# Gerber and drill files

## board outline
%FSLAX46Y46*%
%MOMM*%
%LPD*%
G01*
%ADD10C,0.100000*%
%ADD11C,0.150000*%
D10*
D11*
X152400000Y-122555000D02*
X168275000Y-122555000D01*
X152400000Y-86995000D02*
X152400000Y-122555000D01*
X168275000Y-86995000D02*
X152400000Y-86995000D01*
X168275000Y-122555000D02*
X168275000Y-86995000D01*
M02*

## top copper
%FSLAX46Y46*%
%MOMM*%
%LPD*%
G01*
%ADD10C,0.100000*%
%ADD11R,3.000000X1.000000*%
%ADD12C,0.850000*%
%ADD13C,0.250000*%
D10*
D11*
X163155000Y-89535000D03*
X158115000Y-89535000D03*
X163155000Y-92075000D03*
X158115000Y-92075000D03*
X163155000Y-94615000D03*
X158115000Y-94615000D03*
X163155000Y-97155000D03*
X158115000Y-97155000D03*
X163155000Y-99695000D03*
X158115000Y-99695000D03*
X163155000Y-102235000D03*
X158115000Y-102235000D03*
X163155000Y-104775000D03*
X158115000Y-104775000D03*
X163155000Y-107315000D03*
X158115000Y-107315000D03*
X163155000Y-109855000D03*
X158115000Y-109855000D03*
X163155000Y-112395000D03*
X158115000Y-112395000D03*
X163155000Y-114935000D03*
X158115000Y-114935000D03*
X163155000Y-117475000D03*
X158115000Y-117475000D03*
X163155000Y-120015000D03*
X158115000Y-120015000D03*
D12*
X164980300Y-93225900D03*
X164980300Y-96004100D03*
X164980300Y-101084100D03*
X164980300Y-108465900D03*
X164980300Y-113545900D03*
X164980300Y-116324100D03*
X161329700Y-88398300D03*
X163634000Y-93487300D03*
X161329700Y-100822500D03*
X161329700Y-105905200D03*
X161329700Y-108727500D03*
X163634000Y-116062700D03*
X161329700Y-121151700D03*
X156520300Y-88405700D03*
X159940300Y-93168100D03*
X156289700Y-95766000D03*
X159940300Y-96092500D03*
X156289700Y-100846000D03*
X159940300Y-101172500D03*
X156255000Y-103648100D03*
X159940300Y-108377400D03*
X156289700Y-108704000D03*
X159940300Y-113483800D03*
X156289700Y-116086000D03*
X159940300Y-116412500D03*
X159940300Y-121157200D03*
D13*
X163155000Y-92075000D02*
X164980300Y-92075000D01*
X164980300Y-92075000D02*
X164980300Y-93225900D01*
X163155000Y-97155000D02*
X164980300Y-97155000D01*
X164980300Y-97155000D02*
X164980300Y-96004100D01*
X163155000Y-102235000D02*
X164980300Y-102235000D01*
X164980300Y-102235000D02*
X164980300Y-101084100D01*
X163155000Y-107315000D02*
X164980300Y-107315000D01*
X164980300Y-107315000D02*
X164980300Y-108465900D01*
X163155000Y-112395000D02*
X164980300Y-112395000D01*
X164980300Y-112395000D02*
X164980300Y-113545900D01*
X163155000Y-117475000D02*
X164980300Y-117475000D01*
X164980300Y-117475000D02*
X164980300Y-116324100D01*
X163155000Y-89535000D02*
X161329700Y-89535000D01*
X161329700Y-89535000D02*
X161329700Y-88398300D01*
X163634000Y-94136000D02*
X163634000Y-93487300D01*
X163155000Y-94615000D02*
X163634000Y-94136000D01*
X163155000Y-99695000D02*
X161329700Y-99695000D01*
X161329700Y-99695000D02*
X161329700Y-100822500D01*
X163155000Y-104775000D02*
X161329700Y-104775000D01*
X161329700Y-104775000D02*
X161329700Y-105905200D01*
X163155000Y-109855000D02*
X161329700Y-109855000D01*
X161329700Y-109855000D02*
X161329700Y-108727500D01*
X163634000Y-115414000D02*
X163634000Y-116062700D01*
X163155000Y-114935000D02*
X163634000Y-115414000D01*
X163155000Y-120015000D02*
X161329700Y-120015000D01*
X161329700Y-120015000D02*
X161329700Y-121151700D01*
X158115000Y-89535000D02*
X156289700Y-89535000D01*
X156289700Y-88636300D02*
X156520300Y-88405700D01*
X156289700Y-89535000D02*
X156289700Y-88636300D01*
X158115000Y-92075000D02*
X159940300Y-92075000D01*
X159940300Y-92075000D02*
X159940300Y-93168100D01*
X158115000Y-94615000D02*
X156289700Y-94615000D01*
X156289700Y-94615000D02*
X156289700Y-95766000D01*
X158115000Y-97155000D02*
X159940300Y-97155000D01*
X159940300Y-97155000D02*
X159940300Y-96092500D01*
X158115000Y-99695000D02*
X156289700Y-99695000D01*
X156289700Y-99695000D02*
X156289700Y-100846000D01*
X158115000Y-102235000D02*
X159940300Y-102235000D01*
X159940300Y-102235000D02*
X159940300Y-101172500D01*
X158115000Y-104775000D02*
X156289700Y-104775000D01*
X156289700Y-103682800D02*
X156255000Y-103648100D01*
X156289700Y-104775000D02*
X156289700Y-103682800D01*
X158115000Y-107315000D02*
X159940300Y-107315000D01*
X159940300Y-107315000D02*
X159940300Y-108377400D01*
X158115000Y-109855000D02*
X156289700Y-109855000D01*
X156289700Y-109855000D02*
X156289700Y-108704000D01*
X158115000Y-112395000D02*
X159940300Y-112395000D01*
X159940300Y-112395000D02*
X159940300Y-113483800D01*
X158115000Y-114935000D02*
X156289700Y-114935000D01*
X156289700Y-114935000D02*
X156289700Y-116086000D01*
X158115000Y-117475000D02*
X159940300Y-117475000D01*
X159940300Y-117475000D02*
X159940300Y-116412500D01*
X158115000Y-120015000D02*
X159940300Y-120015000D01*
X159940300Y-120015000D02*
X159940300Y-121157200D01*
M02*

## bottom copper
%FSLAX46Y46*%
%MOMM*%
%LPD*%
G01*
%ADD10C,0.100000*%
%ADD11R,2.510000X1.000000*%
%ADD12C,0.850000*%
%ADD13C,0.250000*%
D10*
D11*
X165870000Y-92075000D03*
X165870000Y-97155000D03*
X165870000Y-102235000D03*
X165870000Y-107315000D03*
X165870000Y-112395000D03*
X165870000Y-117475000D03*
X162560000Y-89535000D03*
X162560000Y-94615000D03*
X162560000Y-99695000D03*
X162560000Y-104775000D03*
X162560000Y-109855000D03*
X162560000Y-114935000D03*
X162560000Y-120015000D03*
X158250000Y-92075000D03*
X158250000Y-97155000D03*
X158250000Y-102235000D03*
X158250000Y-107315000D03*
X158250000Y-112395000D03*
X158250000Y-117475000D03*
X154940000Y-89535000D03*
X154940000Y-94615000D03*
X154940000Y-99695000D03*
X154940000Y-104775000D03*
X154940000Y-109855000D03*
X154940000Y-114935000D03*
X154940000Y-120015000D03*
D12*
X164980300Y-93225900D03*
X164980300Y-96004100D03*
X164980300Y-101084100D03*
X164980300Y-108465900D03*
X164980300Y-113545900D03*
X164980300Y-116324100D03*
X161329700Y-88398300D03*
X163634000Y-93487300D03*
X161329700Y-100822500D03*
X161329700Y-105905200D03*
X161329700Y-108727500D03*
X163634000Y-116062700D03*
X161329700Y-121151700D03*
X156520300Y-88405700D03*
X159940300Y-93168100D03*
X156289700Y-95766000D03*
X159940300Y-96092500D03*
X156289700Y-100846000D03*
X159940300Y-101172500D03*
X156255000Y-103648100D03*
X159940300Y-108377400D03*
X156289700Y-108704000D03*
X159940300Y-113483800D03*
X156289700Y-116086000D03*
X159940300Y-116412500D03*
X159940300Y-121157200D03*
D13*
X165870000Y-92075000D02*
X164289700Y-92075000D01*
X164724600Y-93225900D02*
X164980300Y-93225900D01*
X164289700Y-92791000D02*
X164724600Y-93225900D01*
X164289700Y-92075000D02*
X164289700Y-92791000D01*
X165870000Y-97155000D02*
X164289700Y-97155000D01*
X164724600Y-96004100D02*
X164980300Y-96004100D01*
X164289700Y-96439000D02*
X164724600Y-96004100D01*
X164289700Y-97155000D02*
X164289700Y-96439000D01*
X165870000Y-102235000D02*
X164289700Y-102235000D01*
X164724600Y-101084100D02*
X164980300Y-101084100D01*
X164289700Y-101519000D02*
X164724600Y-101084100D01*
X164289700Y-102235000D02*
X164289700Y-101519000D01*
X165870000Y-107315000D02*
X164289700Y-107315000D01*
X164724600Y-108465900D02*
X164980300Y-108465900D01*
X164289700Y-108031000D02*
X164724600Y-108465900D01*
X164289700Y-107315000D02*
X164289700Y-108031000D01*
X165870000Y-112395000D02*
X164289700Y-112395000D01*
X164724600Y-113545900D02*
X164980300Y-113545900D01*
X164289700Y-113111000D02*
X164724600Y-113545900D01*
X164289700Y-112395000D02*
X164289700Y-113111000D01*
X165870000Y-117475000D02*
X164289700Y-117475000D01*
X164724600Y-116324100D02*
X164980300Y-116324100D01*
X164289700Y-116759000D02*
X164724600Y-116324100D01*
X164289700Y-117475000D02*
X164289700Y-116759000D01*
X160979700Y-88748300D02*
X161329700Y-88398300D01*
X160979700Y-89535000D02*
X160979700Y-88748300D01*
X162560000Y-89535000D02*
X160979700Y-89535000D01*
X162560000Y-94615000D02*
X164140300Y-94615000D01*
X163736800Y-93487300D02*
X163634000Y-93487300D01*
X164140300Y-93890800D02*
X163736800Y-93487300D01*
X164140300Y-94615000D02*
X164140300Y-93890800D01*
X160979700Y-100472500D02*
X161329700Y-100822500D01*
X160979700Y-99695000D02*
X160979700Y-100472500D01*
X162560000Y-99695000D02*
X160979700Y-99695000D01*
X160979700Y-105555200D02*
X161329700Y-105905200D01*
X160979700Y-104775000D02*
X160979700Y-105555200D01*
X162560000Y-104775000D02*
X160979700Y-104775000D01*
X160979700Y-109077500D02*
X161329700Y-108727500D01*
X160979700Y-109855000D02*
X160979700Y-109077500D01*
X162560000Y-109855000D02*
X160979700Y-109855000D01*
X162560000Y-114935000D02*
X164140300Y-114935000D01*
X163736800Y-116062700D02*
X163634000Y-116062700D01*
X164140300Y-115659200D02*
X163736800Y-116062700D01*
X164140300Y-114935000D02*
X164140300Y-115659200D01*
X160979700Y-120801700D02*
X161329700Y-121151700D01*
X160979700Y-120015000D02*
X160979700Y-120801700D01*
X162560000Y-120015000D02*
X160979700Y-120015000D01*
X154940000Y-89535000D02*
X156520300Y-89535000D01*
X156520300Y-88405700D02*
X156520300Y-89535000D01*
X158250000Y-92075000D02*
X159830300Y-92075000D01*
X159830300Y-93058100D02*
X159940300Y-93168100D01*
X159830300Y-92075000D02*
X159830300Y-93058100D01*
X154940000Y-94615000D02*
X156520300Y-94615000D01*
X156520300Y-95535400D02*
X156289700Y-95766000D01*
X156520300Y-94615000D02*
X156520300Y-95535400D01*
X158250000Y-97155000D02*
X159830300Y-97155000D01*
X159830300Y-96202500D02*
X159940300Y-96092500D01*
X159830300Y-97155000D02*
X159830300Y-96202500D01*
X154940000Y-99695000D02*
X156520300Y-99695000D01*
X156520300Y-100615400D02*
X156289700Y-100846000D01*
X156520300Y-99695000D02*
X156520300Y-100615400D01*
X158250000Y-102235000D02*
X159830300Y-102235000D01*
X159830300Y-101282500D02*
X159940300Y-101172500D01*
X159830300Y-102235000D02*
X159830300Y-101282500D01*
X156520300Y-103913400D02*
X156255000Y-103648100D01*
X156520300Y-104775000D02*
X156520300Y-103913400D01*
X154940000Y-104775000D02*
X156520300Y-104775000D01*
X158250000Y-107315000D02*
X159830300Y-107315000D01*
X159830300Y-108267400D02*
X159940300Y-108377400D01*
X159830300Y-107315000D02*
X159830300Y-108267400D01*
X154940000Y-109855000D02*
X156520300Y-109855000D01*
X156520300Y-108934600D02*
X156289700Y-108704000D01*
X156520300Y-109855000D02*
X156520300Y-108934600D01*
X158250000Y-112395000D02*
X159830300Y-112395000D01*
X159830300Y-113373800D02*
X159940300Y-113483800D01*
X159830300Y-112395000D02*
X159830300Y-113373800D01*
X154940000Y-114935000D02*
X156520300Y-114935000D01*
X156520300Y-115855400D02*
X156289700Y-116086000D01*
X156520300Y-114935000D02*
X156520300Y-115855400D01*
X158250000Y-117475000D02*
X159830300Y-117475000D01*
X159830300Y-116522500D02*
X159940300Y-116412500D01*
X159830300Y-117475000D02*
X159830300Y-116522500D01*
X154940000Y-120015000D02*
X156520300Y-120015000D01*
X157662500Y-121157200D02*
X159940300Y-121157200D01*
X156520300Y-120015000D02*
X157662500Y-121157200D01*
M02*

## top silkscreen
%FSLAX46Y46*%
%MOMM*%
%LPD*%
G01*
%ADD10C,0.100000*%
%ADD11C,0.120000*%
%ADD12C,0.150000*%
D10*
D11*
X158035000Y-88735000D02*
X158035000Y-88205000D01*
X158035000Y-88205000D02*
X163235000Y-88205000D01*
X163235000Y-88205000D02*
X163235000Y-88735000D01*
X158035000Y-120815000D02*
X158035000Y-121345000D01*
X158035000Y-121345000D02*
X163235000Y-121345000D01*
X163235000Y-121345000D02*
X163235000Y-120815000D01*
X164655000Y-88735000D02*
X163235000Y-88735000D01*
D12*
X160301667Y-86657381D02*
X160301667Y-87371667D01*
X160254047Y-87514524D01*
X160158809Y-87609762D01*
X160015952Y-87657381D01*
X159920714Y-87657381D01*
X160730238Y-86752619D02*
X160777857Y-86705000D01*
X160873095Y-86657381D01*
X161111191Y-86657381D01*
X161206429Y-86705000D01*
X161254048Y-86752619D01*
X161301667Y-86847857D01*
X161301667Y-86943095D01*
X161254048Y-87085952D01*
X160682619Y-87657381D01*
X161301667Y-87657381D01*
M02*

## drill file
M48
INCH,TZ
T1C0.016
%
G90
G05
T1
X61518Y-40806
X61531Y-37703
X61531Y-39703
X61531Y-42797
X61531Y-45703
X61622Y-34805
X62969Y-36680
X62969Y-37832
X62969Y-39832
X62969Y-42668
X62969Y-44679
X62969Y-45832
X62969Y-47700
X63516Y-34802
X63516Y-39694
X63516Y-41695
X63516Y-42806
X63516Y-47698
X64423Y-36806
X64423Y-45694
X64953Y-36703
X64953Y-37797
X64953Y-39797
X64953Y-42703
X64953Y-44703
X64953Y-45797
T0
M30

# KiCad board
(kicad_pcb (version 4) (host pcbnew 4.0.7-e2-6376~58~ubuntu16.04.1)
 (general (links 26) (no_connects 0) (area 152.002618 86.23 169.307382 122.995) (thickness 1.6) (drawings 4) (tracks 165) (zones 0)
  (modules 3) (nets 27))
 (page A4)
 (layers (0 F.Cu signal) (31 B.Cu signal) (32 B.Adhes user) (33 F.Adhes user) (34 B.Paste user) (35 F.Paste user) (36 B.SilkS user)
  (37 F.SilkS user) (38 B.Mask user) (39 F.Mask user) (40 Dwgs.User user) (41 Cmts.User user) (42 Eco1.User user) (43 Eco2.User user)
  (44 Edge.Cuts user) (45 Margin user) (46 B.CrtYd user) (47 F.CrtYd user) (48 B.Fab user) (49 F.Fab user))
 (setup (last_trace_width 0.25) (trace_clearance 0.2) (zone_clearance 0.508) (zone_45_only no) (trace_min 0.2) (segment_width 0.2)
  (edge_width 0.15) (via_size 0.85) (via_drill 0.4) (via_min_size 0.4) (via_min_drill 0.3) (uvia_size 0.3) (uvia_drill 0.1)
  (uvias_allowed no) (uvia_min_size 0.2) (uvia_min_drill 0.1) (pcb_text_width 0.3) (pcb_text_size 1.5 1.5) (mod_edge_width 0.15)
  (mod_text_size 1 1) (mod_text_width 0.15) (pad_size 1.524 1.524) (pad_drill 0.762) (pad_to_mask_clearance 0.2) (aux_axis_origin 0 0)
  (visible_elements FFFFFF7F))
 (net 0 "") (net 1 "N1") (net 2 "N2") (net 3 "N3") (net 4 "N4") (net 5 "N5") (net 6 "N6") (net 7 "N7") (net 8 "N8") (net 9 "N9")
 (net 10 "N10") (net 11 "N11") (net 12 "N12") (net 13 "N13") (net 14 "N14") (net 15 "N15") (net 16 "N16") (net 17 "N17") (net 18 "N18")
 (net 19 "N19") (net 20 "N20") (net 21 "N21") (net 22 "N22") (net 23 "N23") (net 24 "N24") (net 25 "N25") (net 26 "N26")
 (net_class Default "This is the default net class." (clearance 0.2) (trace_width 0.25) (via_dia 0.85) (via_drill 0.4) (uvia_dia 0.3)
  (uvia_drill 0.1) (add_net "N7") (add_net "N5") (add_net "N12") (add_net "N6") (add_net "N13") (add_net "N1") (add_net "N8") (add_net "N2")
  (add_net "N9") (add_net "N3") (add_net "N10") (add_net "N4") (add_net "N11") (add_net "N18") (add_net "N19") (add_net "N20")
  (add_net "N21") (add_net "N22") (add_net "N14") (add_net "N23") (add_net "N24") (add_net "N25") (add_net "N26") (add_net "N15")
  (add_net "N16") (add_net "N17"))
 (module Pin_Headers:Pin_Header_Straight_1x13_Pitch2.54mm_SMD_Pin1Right (layer B.Cu) (at 164.215 104.775 180)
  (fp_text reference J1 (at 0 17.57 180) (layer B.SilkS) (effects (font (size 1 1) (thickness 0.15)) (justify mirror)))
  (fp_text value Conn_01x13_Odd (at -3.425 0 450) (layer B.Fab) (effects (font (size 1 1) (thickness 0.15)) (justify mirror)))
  (pad 2 smd rect (at -1.655 12.7 180) (size 2.51 1) (layers B.Cu B.Paste B.Mask) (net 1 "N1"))
  (pad 4 smd rect (at -1.655 7.62 180) (size 2.51 1) (layers B.Cu B.Paste B.Mask) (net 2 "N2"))
  (pad 6 smd rect (at -1.655 2.54 180) (size 2.51 1) (layers B.Cu B.Paste B.Mask) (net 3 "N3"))
  (pad 8 smd rect (at -1.655 -2.54 180) (size 2.51 1) (layers B.Cu B.Paste B.Mask) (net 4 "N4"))
  (pad 10 smd rect (at -1.655 -7.62 180) (size 2.51 1) (layers B.Cu B.Paste B.Mask) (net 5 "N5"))
  (pad 12 smd rect (at -1.655 -12.7 180) (size 2.51 1) (layers B.Cu B.Paste B.Mask) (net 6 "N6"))
  (pad 1 smd rect (at 1.655 15.24 180) (size 2.51 1) (layers B.Cu B.Paste B.Mask) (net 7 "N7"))
  (pad 3 smd rect (at 1.655 10.16 180) (size 2.51 1) (layers B.Cu B.Paste B.Mask) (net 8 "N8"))
  (pad 5 smd rect (at 1.655 5.08 180) (size 2.51 1) (layers B.Cu B.Paste B.Mask) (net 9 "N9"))
  (pad 7 smd rect (at 1.655 0 180) (size 2.51 1) (layers B.Cu B.Paste B.Mask) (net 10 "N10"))
  (pad 9 smd rect (at 1.655 -5.08 180) (size 2.51 1) (layers B.Cu B.Paste B.Mask) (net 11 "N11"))
  (pad 11 smd rect (at 1.655 -10.16 180) (size 2.51 1) (layers B.Cu B.Paste B.Mask) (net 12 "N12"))
  (pad 13 smd rect (at 1.655 -15.24 180) (size 2.51 1) (layers B.Cu B.Paste B.Mask) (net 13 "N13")))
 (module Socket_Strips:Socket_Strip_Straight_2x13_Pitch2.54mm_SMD (layer F.Cu) (at 160.635 104.775)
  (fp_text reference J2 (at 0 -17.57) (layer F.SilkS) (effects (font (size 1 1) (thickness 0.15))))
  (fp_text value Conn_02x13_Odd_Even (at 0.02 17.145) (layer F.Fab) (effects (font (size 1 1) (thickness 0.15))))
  (fp_line (start -2.6 -16.04) (end -2.6 -16.57) (layer F.SilkS) (width 0.12))
  (fp_line (start -2.6 -16.57) (end 2.6 -16.57) (layer F.SilkS) (width 0.12))
  (fp_line (start 2.6 -16.57) (end 2.6 -16.04) (layer F.SilkS) (width 0.12))
  (fp_line (start -2.6 16.04) (end -2.6 16.57) (layer F.SilkS) (width 0.12))
  (fp_line (start -2.6 16.57) (end 2.6 16.57) (layer F.SilkS) (width 0.12))
  (fp_line (start 2.6 16.57) (end 2.6 16.04) (layer F.SilkS) (width 0.12))
  (fp_line (start 4.02 -16.04) (end 2.6 -16.04) (layer F.SilkS) (width 0.12))
  (pad 1 smd rect (at 2.52 -15.24) (size 3 1) (layers F.Cu F.Paste F.Mask) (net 7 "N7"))
  (pad 2 smd rect (at -2.52 -15.24) (size 3 1) (layers F.Cu F.Paste F.Mask) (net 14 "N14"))
  (pad 3 smd rect (at 2.52 -12.7) (size 3 1) (layers F.Cu F.Paste F.Mask) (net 1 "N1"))
  (pad 4 smd rect (at -2.52 -12.7) (size 3 1) (layers F.Cu F.Paste F.Mask) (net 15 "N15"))
  (pad 5 smd rect (at 2.52 -10.16) (size 3 1) (layers F.Cu F.Paste F.Mask) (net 8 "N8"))
  (pad 6 smd rect (at -2.52 -10.16) (size 3 1) (layers F.Cu F.Paste F.Mask) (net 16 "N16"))
  (pad 7 smd rect (at 2.52 -7.62) (size 3 1) (layers F.Cu F.Paste F.Mask) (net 2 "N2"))
  (pad 8 smd rect (at -2.52 -7.62) (size 3 1) (layers F.Cu F.Paste F.Mask) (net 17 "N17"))
  (pad 9 smd rect (at 2.52 -5.08) (size 3 1) (layers F.Cu F.Paste F.Mask) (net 9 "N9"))
  (pad 10 smd rect (at -2.52 -5.08) (size 3 1) (layers F.Cu F.Paste F.Mask) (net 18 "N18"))
  (pad 11 smd rect (at 2.52 -2.54) (size 3 1) (layers F.Cu F.Paste F.Mask) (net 3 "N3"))
  (pad 12 smd rect (at -2.52 -2.54) (size 3 1) (layers F.Cu F.Paste F.Mask) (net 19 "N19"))
  (pad 13 smd rect (at 2.52 0) (size 3 1) (layers F.Cu F.Paste F.Mask) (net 10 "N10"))
  (pad 14 smd rect (at -2.52 0) (size 3 1) (layers F.Cu F.Paste F.Mask) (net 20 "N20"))
  (pad 15 smd rect (at 2.52 2.54) (size 3 1) (layers F.Cu F.Paste F.Mask) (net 4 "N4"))
  (pad 16 smd rect (at -2.52 2.54) (size 3 1) (layers F.Cu F.Paste F.Mask) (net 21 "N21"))
  (pad 17 smd rect (at 2.52 5.08) (size 3 1) (layers F.Cu F.Paste F.Mask) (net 11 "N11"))
  (pad 18 smd rect (at -2.52 5.08) (size 3 1) (layers F.Cu F.Paste F.Mask) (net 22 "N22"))
  (pad 19 smd rect (at 2.52 7.62) (size 3 1) (layers F.Cu F.Paste F.Mask) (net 5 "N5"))
  (pad 20 smd rect (at -2.52 7.62) (size 3 1) (layers F.Cu F.Paste F.Mask) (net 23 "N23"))
  (pad 21 smd rect (at 2.52 10.16) (size 3 1) (layers F.Cu F.Paste F.Mask) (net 12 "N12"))
  (pad 22 smd rect (at -2.52 10.16) (size 3 1) (layers F.Cu F.Paste F.Mask) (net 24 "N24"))
  (pad 23 smd rect (at 2.52 12.7) (size 3 1) (layers F.Cu F.Paste F.Mask) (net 6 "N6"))
  (pad 24 smd rect (at -2.52 12.7) (size 3 1) (layers F.Cu F.Paste F.Mask) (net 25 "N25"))
  (pad 25 smd rect (at 2.52 15.24) (size 3 1) (layers F.Cu F.Paste F.Mask) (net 13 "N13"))
  (pad 26 smd rect (at -2.52 15.24) (size 3 1) (layers F.Cu F.Paste F.Mask) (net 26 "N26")))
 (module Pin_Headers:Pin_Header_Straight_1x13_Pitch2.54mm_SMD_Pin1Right (layer B.Cu) (at 156.595 104.775 180)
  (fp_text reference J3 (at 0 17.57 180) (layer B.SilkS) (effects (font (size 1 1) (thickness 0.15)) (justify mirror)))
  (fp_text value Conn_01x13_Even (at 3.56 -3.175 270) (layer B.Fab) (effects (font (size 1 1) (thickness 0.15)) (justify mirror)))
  (pad 2 smd rect (at -1.655 12.7 180) (size 2.51 1) (layers B.Cu B.Paste B.Mask) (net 15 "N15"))
  (pad 4 smd rect (at -1.655 7.62 180) (size 2.51 1) (layers B.Cu B.Paste B.Mask) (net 17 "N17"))
  (pad 6 smd rect (at -1.655 2.54 180) (size 2.51 1) (layers B.Cu B.Paste B.Mask) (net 19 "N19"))
  (pad 8 smd rect (at -1.655 -2.54 180) (size 2.51 1) (layers B.Cu B.Paste B.Mask) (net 21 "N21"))
  (pad 10 smd rect (at -1.655 -7.62 180) (size 2.51 1) (layers B.Cu B.Paste B.Mask) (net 23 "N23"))
  (pad 12 smd rect (at -1.655 -12.7 180) (size 2.51 1) (layers B.Cu B.Paste B.Mask) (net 25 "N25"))
  (pad 1 smd rect (at 1.655 15.24 180) (size 2.51 1) (layers B.Cu B.Paste B.Mask) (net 14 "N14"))
  (pad 3 smd rect (at 1.655 10.16 180) (size 2.51 1) (layers B.Cu B.Paste B.Mask) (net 16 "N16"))
  (pad 5 smd rect (at 1.655 5.08 180) (size 2.51 1) (layers B.Cu B.Paste B.Mask) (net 18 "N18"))
  (pad 7 smd rect (at 1.655 0 180) (size 2.51 1) (layers B.Cu B.Paste B.Mask) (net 20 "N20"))
  (pad 9 smd rect (at 1.655 -5.08 180) (size 2.51 1) (layers B.Cu B.Paste B.Mask) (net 22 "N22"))
  (pad 11 smd rect (at 1.655 -10.16 180) (size 2.51 1) (layers B.Cu B.Paste B.Mask) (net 24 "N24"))
  (pad 13 smd rect (at 1.655 -15.24 180) (size 2.51 1) (layers B.Cu B.Paste B.Mask) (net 26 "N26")))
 (gr_line (start 152.4 122.555) (end 168.275 122.555) (layer Edge.Cuts) (width 0.15))
 (gr_line (start 152.4 86.995) (end 152.4 122.555) (layer Edge.Cuts) (width 0.15))
 (gr_line (start 168.275 86.995) (end 152.4 86.995) (layer Edge.Cuts) (width 0.15))
 (gr_line (start 168.275 122.555) (end 168.275 86.995) (layer Edge.Cuts) (width 0.15))
 (via (at 164.9803 93.2259) (size 0.85) (layers F.Cu B.Cu) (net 1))
 (segment (start 163.155 92.075) (end 164.9803 92.075) (width 0.25) (layer F.Cu) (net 1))
 (segment (start 165.87 92.075) (end 164.2897 92.075) (width 0.25) (layer B.Cu) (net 1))
 (segment (start 164.7246 93.2259) (end 164.9803 93.2259) (width 0.25) (layer B.Cu) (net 1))
 (segment (start 164.2897 92.791) (end 164.7246 93.2259) (width 0.25) (layer B.Cu) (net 1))
 (segment (start 164.2897 92.075) (end 164.2897 92.791) (width 0.25) (layer B.Cu) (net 1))
 (segment (start 164.9803 92.075) (end 164.9803 93.2259) (width 0.25) (layer F.Cu) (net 1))
 (via (at 164.9803 96.0041) (size 0.85) (layers F.Cu B.Cu) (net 2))
 (segment (start 163.155 97.155) (end 164.9803 97.155) (width 0.25) (layer F.Cu) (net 2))
 (segment (start 165.87 97.155) (end 164.2897 97.155) (width 0.25) (layer B.Cu) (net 2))
 (segment (start 164.7246 96.0041) (end 164.9803 96.0041) (width 0.25) (layer B.Cu) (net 2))
 (segment (start 164.2897 96.439) (end 164.7246 96.0041) (width 0.25) (layer B.Cu) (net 2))
 (segment (start 164.2897 97.155) (end 164.2897 96.439) (width 0.25) (layer B.Cu) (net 2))
 (segment (start 164.9803 97.155) (end 164.9803 96.0041) (width 0.25) (layer F.Cu) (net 2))
 (via (at 164.9803 101.0841) (size 0.85) (layers F.Cu B.Cu) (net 3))
 (segment (start 163.155 102.235) (end 164.9803 102.235) (width 0.25) (layer F.Cu) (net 3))
 (segment (start 165.87 102.235) (end 164.2897 102.235) (width 0.25) (layer B.Cu) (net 3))
 (segment (start 164.7246 101.0841) (end 164.9803 101.0841) (width 0.25) (layer B.Cu) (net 3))
 (segment (start 164.2897 101.519) (end 164.7246 101.0841) (width 0.25) (layer B.Cu) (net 3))
 (segment (start 164.2897 102.235) (end 164.2897 101.519) (width 0.25) (layer B.Cu) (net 3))
 (segment (start 164.9803 102.235) (end 164.9803 101.0841) (width 0.25) (layer F.Cu) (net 3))
 (via (at 164.9803 108.4659) (size 0.85) (layers F.Cu B.Cu) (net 4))
 (segment (start 163.155 107.315) (end 164.9803 107.315) (width 0.25) (layer F.Cu) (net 4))
 (segment (start 165.87 107.315) (end 164.2897 107.315) (width 0.25) (layer B.Cu) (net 4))
 (segment (start 164.7246 108.4659) (end 164.9803 108.4659) (width 0.25) (layer B.Cu) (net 4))
 (segment (start 164.2897 108.031) (end 164.7246 108.4659) (width 0.25) (layer B.Cu) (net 4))
 (segment (start 164.2897 107.315) (end 164.2897 108.031) (width 0.25) (layer B.Cu) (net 4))
 (segment (start 164.9803 107.315) (end 164.9803 108.4659) (width 0.25) (layer F.Cu) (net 4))
 (via (at 164.9803 113.5459) (size 0.85) (layers F.Cu B.Cu) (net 5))
 (segment (start 163.155 112.395) (end 164.9803 112.395) (width 0.25) (layer F.Cu) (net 5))
 (segment (start 165.87 112.395) (end 164.2897 112.395) (width 0.25) (layer B.Cu) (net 5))
 (segment (start 164.7246 113.5459) (end 164.9803 113.5459) (width 0.25) (layer B.Cu) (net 5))
 (segment (start 164.2897 113.111) (end 164.7246 113.5459) (width 0.25) (layer B.Cu) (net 5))
 (segment (start 164.2897 112.395) (end 164.2897 113.111) (width 0.25) (layer B.Cu) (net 5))
 (segment (start 164.9803 112.395) (end 164.9803 113.5459) (width 0.25) (layer F.Cu) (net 5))
 (via (at 164.9803 116.3241) (size 0.85) (layers F.Cu B.Cu) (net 6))
 (segment (start 163.155 117.475) (end 164.9803 117.475) (width 0.25) (layer F.Cu) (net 6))
 (segment (start 165.87 117.475) (end 164.2897 117.475) (width 0.25) (layer B.Cu) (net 6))
 (segment (start 164.7246 116.3241) (end 164.9803 116.3241) (width 0.25) (layer B.Cu) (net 6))
 (segment (start 164.2897 116.759) (end 164.7246 116.3241) (width 0.25) (layer B.Cu) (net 6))
 (segment (start 164.2897 117.475) (end 164.2897 116.759) (width 0.25) (layer B.Cu) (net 6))
 (segment (start 164.9803 117.475) (end 164.9803 116.3241) (width 0.25) (layer F.Cu) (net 6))
 (via (at 161.3297 88.3983) (size 0.85) (layers F.Cu B.Cu) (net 7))
 (segment (start 163.155 89.535) (end 161.3297 89.535) (width 0.25) (layer F.Cu) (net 7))
 (segment (start 160.9797 88.7483) (end 161.3297 88.3983) (width 0.25) (layer B.Cu) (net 7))
 (segment (start 160.9797 89.535) (end 160.9797 88.7483) (width 0.25) (layer B.Cu) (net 7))
 (segment (start 161.3297 89.535) (end 161.3297 88.3983) (width 0.25) (layer F.Cu) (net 7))
 (segment (start 162.56 89.535) (end 160.9797 89.535) (width 0.25) (layer B.Cu) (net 7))
 (via (at 163.634 93.4873) (size 0.85) (layers F.Cu B.Cu) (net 8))
 (segment (start 162.56 94.615) (end 164.1403 94.615) (width 0.25) (layer B.Cu) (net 8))
 (segment (start 163.7368 93.4873) (end 163.634 93.4873) (width 0.25) (layer B.Cu) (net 8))
 (segment (start 164.1403 93.8908) (end 163.7368 93.4873) (width 0.25) (layer B.Cu) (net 8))
 (segment (start 164.1403 94.615) (end 164.1403 93.8908) (width 0.25) (layer B.Cu) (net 8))
 (segment (start 163.634 94.136) (end 163.634 93.4873) (width 0.25) (layer F.Cu) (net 8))
 (segment (start 163.155 94.615) (end 163.634 94.136) (width 0.25) (layer F.Cu) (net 8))
 (via (at 161.3297 100.8225) (size 0.85) (layers F.Cu B.Cu) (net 9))
 (segment (start 163.155 99.695) (end 161.3297 99.695) (width 0.25) (layer F.Cu) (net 9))
 (segment (start 160.9797 100.4725) (end 161.3297 100.8225) (width 0.25) (layer B.Cu) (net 9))
 (segment (start 160.9797 99.695) (end 160.9797 100.4725) (width 0.25) (layer B.Cu) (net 9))
 (segment (start 161.3297 99.695) (end 161.3297 100.8225) (width 0.25) (layer F.Cu) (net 9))
 (segment (start 162.56 99.695) (end 160.9797 99.695) (width 0.25) (layer B.Cu) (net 9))
 (via (at 161.3297 105.9052) (size 0.85) (layers F.Cu B.Cu) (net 10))
 (segment (start 163.155 104.775) (end 161.3297 104.775) (width 0.25) (layer F.Cu) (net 10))
 (segment (start 160.9797 105.5552) (end 161.3297 105.9052) (width 0.25) (layer B.Cu) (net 10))
 (segment (start 160.9797 104.775) (end 160.9797 105.5552) (width 0.25) (layer B.Cu) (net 10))
 (segment (start 161.3297 104.775) (end 161.3297 105.9052) (width 0.25) (layer F.Cu) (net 10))
 (segment (start 162.56 104.775) (end 160.9797 104.775) (width 0.25) (layer B.Cu) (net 10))
 (via (at 161.3297 108.7275) (size 0.85) (layers F.Cu B.Cu) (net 11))
 (segment (start 163.155 109.855) (end 161.3297 109.855) (width 0.25) (layer F.Cu) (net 11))
 (segment (start 160.9797 109.0775) (end 161.3297 108.7275) (width 0.25) (layer B.Cu) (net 11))
 (segment (start 160.9797 109.855) (end 160.9797 109.0775) (width 0.25) (layer B.Cu) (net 11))
 (segment (start 161.3297 109.855) (end 161.3297 108.7275) (width 0.25) (layer F.Cu) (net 11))
 (segment (start 162.56 109.855) (end 160.9797 109.855) (width 0.25) (layer B.Cu) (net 11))
 (via (at 163.634 116.0627) (size 0.85) (layers F.Cu B.Cu) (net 12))
 (segment (start 162.56 114.935) (end 164.1403 114.935) (width 0.25) (layer B.Cu) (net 12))
 (segment (start 163.7368 116.0627) (end 163.634 116.0627) (width 0.25) (layer B.Cu) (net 12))
 (segment (start 164.1403 115.6592) (end 163.7368 116.0627) (width 0.25) (layer B.Cu) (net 12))
 (segment (start 164.1403 114.935) (end 164.1403 115.6592) (width 0.25) (layer B.Cu) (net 12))
 (segment (start 163.634 115.414) (end 163.634 116.0627) (width 0.25) (layer F.Cu) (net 12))
 (segment (start 163.155 114.935) (end 163.634 115.414) (width 0.25) (layer F.Cu) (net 12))
 (via (at 161.3297 121.1517) (size 0.85) (layers F.Cu B.Cu) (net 13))
 (segment (start 163.155 120.015) (end 161.3297 120.015) (width 0.25) (layer F.Cu) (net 13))
 (segment (start 160.9797 120.8017) (end 161.3297 121.1517) (width 0.25) (layer B.Cu) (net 13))
 (segment (start 160.9797 120.015) (end 160.9797 120.8017) (width 0.25) (layer B.Cu) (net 13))
 (segment (start 161.3297 120.015) (end 161.3297 121.1517) (width 0.25) (layer F.Cu) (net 13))
 (segment (start 162.56 120.015) (end 160.9797 120.015) (width 0.25) (layer B.Cu) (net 13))
 (via (at 156.5203 88.4057) (size 0.85) (layers F.Cu B.Cu) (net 14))
 (segment (start 158.115 89.535) (end 156.2897 89.535) (width 0.25) (layer F.Cu) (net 14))
 (segment (start 154.94 89.535) (end 156.5203 89.535) (width 0.25) (layer B.Cu) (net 14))
 (segment (start 156.5203 88.4057) (end 156.5203 89.535) (width 0.25) (layer B.Cu) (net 14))
 (segment (start 156.2897 88.6363) (end 156.5203 88.4057) (width 0.25) (layer F.Cu) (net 14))
 (segment (start 156.2897 89.535) (end 156.2897 88.6363) (width 0.25) (layer F.Cu) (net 14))
 (via (at 159.9403 93.1681) (size 0.85) (layers F.Cu B.Cu) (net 15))
 (segment (start 158.115 92.075) (end 159.9403 92.075) (width 0.25) (layer F.Cu) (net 15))
 (segment (start 158.25 92.075) (end 159.8303 92.075) (width 0.25) (layer B.Cu) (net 15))
 (segment (start 159.8303 93.0581) (end 159.9403 93.1681) (width 0.25) (layer B.Cu) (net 15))
 (segment (start 159.8303 92.075) (end 159.8303 93.0581) (width 0.25) (layer B.Cu) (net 15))
 (segment (start 159.9403 92.075) (end 159.9403 93.1681) (width 0.25) (layer F.Cu) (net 15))
 (via (at 156.2897 95.766) (size 0.85) (layers F.Cu B.Cu) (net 16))
 (segment (start 158.115 94.615) (end 156.2897 94.615) (width 0.25) (layer F.Cu) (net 16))
 (segment (start 154.94 94.615) (end 156.5203 94.615) (width 0.25) (layer B.Cu) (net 16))
 (segment (start 156.5203 95.5354) (end 156.2897 95.766) (width 0.25) (layer B.Cu) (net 16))
 (segment (start 156.5203 94.615) (end 156.5203 95.5354) (width 0.25) (layer B.Cu) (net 16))
 (segment (start 156.2897 94.615) (end 156.2897 95.766) (width 0.25) (layer F.Cu) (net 16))
 (via (at 159.9403 96.0925) (size 0.85) (layers F.Cu B.Cu) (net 17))
 (segment (start 158.115 97.155) (end 159.9403 97.155) (width 0.25) (layer F.Cu) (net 17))
 (segment (start 158.25 97.155) (end 159.8303 97.155) (width 0.25) (layer B.Cu) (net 17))
 (segment (start 159.8303 96.2025) (end 159.9403 96.0925) (width 0.25) (layer B.Cu) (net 17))
 (segment (start 159.8303 97.155) (end 159.8303 96.2025) (width 0.25) (layer B.Cu) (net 17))
 (segment (start 159.9403 97.155) (end 159.9403 96.0925) (width 0.25) (layer F.Cu) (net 17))
 (via (at 156.2897 100.846) (size 0.85) (layers F.Cu B.Cu) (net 18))
 (segment (start 158.115 99.695) (end 156.2897 99.695) (width 0.25) (layer F.Cu) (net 18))
 (segment (start 154.94 99.695) (end 156.5203 99.695) (width 0.25) (layer B.Cu) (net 18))
 (segment (start 156.5203 100.6154) (end 156.2897 100.846) (width 0.25) (layer B.Cu) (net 18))
 (segment (start 156.5203 99.695) (end 156.5203 100.6154) (width 0.25) (layer B.Cu) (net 18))
 (segment (start 156.2897 99.695) (end 156.2897 100.846) (width 0.25) (layer F.Cu) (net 18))
 (via (at 159.9403 101.1725) (size 0.85) (layers F.Cu B.Cu) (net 19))
 (segment (start 158.115 102.235) (end 159.9403 102.235) (width 0.25) (layer F.Cu) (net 19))
 (segment (start 158.25 102.235) (end 159.8303 102.235) (width 0.25) (layer B.Cu) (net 19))
 (segment (start 159.8303 101.2825) (end 159.9403 101.1725) (width 0.25) (layer B.Cu) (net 19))
 (segment (start 159.8303 102.235) (end 159.8303 101.2825) (width 0.25) (layer B.Cu) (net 19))
 (segment (start 159.9403 102.235) (end 159.9403 101.1725) (width 0.25) (layer F.Cu) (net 19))
 (via (at 156.255 103.6481) (size 0.85) (layers F.Cu B.Cu) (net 20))
 (segment (start 158.115 104.775) (end 156.2897 104.775) (width 0.25) (layer F.Cu) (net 20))
 (segment (start 156.5203 103.9134) (end 156.255 103.6481) (width 0.25) (layer B.Cu) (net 20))
 (segment (start 156.5203 104.775) (end 156.5203 103.9134) (width 0.25) (layer B.Cu) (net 20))
 (segment (start 156.2897 103.6828) (end 156.255 103.6481) (width 0.25) (layer F.Cu) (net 20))
 (segment (start 156.2897 104.775) (end 156.2897 103.6828) (width 0.25) (layer F.Cu) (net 20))
 (segment (start 154.94 104.775) (end 156.5203 104.775) (width 0.25) (layer B.Cu) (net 20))
 (via (at 159.9403 108.3774) (size 0.85) (layers F.Cu B.Cu) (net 21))
 (segment (start 158.115 107.315) (end 159.9403 107.315) (width 0.25) (layer F.Cu) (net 21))
 (segment (start 158.25 107.315) (end 159.8303 107.315) (width 0.25) (layer B.Cu) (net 21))
 (segment (start 159.8303 108.2674) (end 159.9403 108.3774) (width 0.25) (layer B.Cu) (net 21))
 (segment (start 159.8303 107.315) (end 159.8303 108.2674) (width 0.25) (layer B.Cu) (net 21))
 (segment (start 159.9403 107.315) (end 159.9403 108.3774) (width 0.25) (layer F.Cu) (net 21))
 (via (at 156.2897 108.704) (size 0.85) (layers F.Cu B.Cu) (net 22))
 (segment (start 158.115 109.855) (end 156.2897 109.855) (width 0.25) (layer F.Cu) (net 22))
 (segment (start 154.94 109.855) (end 156.5203 109.855) (width 0.25) (layer B.Cu) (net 22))
 (segment (start 156.5203 108.9346) (end 156.2897 108.704) (width 0.25) (layer B.Cu) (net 22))
 (segment (start 156.5203 109.855) (end 156.5203 108.9346) (width 0.25) (layer B.Cu) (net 22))
 (segment (start 156.2897 109.855) (end 156.2897 108.704) (width 0.25) (layer F.Cu) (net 22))
 (via (at 159.9403 113.4838) (size 0.85) (layers F.Cu B.Cu) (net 23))
 (segment (start 158.115 112.395) (end 159.9403 112.395) (width 0.25) (layer F.Cu) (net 23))
 (segment (start 158.25 112.395) (end 159.8303 112.395) (width 0.25) (layer B.Cu) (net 23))
 (segment (start 159.8303 113.3738) (end 159.9403 113.4838) (width 0.25) (layer B.Cu) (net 23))
 (segment (start 159.8303 112.395) (end 159.8303 113.3738) (width 0.25) (layer B.Cu) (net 23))
 (segment (start 159.9403 112.395) (end 159.9403 113.4838) (width 0.25) (layer F.Cu) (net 23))
 (via (at 156.2897 116.086) (size 0.85) (layers F.Cu B.Cu) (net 24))
 (segment (start 158.115 114.935) (end 156.2897 114.935) (width 0.25) (layer F.Cu) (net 24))
 (segment (start 154.94 114.935) (end 156.5203 114.935) (width 0.25) (layer B.Cu) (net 24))
 (segment (start 156.5203 115.8554) (end 156.2897 116.086) (width 0.25) (layer B.Cu) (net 24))
 (segment (start 156.5203 114.935) (end 156.5203 115.8554) (width 0.25) (layer B.Cu) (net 24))
 (segment (start 156.2897 114.935) (end 156.2897 116.086) (width 0.25) (layer F.Cu) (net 24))
 (via (at 159.9403 116.4125) (size 0.85) (layers F.Cu B.Cu) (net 25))
 (segment (start 158.115 117.475) (end 159.9403 117.475) (width 0.25) (layer F.Cu) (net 25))
 (segment (start 158.25 117.475) (end 159.8303 117.475) (width 0.25) (layer B.Cu) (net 25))
 (segment (start 159.8303 116.5225) (end 159.9403 116.4125) (width 0.25) (layer B.Cu) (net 25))
 (segment (start 159.8303 117.475) (end 159.8303 116.5225) (width 0.25) (layer B.Cu) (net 25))
 (segment (start 159.9403 117.475) (end 159.9403 116.4125) (width 0.25) (layer F.Cu) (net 25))
 (via (at 159.9403 121.1572) (size 0.85) (layers F.Cu B.Cu) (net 26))
 (segment (start 158.115 120.015) (end 159.9403 120.015) (width 0.25) (layer F.Cu) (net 26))
 (segment (start 154.94 120.015) (end 156.5203 120.015) (width 0.25) (layer B.Cu) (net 26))
 (segment (start 157.6625 121.1572) (end 159.9403 121.1572) (width 0.25) (layer B.Cu) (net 26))
 (segment (start 156.5203 120.015) (end 157.6625 121.1572) (width 0.25) (layer B.Cu) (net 26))
 (segment (start 159.9403 120.015) (end 159.9403 121.1572) (width 0.25) (layer F.Cu) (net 26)))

